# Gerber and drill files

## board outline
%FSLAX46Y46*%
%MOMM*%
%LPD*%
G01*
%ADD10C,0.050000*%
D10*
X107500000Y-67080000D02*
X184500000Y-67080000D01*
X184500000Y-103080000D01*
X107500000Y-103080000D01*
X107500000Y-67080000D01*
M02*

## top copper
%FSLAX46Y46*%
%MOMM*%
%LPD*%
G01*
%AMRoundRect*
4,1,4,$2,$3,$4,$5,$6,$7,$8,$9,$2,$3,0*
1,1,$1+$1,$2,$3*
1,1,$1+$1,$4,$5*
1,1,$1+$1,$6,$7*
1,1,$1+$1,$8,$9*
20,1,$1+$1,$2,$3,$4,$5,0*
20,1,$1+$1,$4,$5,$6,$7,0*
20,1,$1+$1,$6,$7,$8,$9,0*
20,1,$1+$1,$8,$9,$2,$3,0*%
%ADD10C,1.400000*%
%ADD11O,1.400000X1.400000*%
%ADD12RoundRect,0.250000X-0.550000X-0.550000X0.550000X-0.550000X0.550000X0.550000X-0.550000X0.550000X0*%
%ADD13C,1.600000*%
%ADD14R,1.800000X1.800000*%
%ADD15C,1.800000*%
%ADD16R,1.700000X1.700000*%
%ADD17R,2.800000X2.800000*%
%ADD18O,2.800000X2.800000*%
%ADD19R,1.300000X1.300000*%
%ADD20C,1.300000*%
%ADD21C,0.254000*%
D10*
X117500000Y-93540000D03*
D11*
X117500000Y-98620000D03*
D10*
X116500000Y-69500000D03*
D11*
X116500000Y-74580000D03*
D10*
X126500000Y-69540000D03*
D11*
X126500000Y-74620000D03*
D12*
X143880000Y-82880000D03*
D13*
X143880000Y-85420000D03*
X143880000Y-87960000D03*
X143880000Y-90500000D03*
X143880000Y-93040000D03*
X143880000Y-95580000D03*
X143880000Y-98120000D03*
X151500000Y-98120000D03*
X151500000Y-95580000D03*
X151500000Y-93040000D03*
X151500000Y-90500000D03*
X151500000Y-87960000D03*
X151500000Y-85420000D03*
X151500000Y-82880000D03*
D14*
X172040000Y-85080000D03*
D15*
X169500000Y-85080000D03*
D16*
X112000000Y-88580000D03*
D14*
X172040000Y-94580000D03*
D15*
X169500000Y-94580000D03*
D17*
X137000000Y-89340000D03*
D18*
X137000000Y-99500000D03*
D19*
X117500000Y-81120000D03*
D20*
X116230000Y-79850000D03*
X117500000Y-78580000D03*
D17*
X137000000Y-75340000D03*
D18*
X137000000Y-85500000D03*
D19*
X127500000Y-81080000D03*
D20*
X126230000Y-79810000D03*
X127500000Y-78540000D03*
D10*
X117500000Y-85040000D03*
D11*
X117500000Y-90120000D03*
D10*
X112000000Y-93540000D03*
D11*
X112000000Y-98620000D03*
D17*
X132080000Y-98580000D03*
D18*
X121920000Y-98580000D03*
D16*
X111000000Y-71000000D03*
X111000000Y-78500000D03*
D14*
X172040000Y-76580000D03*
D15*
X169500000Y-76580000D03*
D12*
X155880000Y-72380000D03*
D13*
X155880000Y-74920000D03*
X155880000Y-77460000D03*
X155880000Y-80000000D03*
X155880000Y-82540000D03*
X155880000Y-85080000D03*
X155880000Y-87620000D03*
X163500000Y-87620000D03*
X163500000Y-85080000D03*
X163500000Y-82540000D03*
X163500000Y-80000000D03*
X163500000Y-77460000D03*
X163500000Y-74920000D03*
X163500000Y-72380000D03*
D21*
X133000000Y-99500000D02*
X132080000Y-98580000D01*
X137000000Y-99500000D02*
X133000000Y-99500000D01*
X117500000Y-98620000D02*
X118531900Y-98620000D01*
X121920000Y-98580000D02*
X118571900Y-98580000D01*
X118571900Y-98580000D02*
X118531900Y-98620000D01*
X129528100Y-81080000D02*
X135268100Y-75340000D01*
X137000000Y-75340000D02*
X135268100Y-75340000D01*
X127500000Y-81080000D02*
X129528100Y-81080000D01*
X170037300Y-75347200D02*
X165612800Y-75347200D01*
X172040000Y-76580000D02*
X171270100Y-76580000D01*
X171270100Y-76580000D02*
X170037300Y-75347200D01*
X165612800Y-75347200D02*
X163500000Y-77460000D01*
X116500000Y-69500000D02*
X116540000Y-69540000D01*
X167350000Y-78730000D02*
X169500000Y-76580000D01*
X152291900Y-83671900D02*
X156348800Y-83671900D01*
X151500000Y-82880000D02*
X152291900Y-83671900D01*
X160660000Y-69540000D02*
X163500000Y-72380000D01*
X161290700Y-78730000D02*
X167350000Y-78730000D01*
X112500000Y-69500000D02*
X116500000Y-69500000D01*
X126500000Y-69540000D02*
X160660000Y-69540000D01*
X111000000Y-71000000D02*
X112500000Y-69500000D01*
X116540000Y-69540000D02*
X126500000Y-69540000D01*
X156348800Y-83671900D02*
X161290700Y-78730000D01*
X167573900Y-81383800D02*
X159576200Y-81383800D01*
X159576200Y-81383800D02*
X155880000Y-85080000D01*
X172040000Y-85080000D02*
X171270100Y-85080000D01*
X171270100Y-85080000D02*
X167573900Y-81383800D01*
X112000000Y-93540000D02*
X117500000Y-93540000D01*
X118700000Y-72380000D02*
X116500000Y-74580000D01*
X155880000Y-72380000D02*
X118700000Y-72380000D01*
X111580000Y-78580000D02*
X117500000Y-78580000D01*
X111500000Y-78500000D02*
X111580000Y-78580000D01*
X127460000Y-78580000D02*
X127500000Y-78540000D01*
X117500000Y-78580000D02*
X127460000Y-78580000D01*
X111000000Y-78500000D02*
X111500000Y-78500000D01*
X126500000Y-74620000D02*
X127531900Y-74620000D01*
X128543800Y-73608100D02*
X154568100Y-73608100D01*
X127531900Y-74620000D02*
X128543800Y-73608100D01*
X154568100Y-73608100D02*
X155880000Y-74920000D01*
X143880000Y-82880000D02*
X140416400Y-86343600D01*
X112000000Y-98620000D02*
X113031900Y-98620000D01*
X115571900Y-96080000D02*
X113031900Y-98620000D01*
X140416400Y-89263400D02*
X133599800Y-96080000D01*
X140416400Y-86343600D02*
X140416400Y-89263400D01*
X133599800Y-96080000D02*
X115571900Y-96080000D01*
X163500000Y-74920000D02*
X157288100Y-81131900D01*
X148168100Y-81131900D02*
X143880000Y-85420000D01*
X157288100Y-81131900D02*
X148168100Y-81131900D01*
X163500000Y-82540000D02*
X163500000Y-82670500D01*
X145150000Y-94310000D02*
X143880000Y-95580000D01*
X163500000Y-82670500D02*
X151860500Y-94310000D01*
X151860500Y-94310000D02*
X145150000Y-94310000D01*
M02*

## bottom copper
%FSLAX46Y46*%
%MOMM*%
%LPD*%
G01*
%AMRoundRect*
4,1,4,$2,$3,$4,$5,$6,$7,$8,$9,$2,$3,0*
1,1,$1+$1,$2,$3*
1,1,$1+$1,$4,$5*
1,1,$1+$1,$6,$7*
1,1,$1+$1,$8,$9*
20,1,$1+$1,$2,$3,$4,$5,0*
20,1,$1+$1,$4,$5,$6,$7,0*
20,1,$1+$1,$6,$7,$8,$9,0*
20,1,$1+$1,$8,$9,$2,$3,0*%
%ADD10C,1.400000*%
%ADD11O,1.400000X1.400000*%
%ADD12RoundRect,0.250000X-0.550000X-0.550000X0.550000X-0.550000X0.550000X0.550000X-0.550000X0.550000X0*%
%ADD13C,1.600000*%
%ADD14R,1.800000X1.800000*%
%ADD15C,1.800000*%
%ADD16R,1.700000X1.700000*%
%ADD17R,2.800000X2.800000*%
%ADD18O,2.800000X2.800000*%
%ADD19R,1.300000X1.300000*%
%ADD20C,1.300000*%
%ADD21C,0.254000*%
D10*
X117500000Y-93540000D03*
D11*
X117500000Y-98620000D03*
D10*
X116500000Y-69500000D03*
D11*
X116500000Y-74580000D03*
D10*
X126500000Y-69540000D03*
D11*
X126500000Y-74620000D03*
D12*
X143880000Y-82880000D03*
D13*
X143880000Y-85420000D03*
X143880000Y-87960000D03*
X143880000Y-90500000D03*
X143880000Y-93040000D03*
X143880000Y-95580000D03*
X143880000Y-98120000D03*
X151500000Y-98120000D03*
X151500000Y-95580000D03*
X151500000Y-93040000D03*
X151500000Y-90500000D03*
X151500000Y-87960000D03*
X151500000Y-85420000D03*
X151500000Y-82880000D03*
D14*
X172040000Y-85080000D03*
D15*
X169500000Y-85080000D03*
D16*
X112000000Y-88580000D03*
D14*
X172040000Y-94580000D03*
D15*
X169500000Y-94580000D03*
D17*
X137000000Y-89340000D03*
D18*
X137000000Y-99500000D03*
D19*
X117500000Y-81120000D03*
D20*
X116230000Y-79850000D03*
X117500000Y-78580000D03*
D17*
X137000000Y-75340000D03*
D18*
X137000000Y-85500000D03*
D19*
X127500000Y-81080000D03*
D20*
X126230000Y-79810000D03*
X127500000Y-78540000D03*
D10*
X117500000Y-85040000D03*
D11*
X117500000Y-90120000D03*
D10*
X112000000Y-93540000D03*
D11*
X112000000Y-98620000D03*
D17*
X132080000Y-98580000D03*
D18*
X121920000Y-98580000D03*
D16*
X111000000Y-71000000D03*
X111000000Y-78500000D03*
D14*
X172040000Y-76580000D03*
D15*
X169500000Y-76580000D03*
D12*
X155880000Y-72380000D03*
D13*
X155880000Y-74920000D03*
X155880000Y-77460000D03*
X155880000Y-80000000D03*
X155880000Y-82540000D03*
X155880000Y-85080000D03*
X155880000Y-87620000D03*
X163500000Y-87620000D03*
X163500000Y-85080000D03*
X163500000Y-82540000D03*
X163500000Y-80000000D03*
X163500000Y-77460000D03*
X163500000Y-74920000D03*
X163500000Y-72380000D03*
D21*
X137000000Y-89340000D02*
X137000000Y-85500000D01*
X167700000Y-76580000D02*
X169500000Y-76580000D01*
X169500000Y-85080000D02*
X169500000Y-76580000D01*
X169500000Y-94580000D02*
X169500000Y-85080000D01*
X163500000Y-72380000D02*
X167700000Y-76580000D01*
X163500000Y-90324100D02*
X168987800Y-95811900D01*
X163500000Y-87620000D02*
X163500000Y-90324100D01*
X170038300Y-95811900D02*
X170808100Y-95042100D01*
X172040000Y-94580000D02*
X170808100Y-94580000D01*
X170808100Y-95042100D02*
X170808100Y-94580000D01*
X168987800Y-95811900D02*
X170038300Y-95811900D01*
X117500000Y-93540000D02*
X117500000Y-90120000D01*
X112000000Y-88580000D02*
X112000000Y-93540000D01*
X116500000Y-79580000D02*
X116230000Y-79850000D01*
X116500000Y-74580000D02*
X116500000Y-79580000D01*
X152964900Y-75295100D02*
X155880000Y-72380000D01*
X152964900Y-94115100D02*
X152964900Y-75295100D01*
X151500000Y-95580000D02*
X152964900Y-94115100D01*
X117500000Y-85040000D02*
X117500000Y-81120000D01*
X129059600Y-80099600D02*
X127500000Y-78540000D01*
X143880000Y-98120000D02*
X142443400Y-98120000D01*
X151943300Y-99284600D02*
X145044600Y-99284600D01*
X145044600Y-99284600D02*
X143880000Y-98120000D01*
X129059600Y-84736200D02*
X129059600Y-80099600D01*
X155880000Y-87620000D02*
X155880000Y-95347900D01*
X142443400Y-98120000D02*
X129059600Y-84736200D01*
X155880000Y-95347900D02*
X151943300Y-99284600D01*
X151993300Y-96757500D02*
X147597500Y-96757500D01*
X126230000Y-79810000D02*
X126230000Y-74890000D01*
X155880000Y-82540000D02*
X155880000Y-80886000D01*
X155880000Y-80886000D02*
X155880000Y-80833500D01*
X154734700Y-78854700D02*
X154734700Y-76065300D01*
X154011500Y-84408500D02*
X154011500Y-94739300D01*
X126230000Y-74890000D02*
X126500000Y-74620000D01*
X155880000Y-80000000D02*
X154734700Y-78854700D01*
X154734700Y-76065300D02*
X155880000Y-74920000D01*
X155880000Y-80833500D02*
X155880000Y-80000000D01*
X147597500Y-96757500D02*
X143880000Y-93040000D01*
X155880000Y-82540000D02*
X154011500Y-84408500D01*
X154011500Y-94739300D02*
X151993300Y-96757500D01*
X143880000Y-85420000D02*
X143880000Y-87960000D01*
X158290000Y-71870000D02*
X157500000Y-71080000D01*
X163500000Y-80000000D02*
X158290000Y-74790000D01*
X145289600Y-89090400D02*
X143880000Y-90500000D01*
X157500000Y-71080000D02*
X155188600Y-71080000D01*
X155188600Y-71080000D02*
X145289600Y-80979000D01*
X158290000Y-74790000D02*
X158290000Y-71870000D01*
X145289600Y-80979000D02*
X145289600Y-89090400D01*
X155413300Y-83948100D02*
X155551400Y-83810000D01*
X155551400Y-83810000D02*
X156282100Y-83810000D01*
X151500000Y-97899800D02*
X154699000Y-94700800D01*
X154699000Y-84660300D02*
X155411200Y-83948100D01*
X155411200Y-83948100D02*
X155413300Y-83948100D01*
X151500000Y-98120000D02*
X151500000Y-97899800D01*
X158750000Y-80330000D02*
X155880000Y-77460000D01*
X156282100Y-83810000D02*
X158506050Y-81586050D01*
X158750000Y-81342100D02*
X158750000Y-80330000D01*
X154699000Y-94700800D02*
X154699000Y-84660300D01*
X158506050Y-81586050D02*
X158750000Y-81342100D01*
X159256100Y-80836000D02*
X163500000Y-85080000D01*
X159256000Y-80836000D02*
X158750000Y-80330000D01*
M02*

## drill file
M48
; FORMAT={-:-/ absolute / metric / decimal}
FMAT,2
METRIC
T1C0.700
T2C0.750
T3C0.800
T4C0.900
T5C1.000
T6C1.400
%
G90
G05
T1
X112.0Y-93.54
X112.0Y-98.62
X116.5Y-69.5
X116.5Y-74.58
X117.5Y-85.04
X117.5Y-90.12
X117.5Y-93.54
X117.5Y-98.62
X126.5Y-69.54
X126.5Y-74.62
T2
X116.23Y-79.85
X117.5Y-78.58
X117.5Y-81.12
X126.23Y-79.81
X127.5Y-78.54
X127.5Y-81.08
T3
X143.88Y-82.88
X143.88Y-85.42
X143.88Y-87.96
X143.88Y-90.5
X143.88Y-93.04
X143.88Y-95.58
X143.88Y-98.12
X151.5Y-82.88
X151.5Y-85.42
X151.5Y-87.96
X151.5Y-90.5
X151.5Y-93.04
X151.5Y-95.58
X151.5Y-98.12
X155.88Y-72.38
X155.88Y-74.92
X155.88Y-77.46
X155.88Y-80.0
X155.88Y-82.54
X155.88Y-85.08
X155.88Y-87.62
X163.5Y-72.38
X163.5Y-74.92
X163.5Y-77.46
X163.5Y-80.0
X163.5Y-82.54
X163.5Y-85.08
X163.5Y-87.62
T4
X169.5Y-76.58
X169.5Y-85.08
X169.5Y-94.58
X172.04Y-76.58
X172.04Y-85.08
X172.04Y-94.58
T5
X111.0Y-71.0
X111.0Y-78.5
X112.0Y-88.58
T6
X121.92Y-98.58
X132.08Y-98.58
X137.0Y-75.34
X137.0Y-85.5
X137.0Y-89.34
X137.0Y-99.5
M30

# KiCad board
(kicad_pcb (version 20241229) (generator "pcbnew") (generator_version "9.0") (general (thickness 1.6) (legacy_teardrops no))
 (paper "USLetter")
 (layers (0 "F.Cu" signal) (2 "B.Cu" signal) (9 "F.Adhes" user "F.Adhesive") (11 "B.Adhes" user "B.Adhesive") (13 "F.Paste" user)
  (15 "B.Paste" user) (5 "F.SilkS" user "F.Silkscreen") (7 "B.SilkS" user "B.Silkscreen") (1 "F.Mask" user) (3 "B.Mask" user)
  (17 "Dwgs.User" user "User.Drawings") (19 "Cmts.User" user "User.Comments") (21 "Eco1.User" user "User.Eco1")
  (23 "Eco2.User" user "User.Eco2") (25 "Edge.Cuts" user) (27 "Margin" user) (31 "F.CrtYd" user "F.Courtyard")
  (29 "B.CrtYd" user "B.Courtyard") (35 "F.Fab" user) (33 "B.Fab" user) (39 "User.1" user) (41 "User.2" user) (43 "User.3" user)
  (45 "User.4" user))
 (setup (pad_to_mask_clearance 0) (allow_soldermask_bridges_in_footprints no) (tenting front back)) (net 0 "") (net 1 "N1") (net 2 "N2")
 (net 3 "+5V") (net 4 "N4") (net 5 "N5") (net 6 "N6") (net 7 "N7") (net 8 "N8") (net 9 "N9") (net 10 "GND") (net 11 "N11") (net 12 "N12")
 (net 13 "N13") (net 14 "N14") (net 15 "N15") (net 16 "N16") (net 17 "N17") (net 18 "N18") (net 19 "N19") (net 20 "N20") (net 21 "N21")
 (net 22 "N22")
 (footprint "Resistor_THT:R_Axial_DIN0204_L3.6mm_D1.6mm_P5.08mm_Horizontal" (layer "F.Cu") (at 117.5 93.54 -90)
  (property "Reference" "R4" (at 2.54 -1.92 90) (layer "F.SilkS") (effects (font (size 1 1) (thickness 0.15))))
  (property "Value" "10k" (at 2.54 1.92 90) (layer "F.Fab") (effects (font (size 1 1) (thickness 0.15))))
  (pad "1" thru_hole circle (at 0 0 270) (size 1.4 1.4) (drill 0.7) (layers "*.Cu" "*.Mask") (remove_unused_layers no) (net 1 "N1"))
  (pad "2" thru_hole oval (at 5.08 0 270) (size 1.4 1.4) (drill 0.7) (layers "*.Cu" "*.Mask") (remove_unused_layers no) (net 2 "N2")))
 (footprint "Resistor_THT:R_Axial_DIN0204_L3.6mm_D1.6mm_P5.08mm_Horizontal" (layer "F.Cu") (at 116.5 69.5 -90)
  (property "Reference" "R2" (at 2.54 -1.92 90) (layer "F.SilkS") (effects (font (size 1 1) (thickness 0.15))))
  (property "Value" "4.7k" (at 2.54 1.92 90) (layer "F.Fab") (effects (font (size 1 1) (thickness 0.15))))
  (pad "1" thru_hole circle (at 0 0 270) (size 1.4 1.4) (drill 0.7) (layers "*.Cu" "*.Mask") (remove_unused_layers no) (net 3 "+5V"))
  (pad "2" thru_hole oval (at 5.08 0 270) (size 1.4 1.4) (drill 0.7) (layers "*.Cu" "*.Mask") (remove_unused_layers no) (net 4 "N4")))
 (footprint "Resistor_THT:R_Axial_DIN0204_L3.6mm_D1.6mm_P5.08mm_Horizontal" (layer "F.Cu") (at 126.5 69.54 -90)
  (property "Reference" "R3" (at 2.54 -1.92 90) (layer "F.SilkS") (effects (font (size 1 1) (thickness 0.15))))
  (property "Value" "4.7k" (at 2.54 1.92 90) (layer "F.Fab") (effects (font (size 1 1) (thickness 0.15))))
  (pad "1" thru_hole circle (at 0 0 270) (size 1.4 1.4) (drill 0.7) (layers "*.Cu" "*.Mask") (remove_unused_layers no) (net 3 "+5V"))
  (pad "2" thru_hole oval (at 5.08 0 270) (size 1.4 1.4) (drill 0.7) (layers "*.Cu" "*.Mask") (remove_unused_layers no) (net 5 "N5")))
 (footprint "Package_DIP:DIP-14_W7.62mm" (layer "F.Cu") (at 143.88 82.88)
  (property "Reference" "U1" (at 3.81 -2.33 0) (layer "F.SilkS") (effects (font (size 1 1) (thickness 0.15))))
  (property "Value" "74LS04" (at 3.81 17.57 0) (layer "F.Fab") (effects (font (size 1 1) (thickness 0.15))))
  (pad "1" thru_hole roundrect (at 0 0) (size 1.6 1.6) (drill 0.8) (layers "*.Cu" "*.Mask") (remove_unused_layers no)
   (roundrect_rratio 0.15625) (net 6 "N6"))
  (pad "2" thru_hole circle (at 0 2.54) (size 1.6 1.6) (drill 0.8) (layers "*.Cu" "*.Mask") (remove_unused_layers no) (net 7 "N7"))
  (pad "3" thru_hole circle (at 0 5.08) (size 1.6 1.6) (drill 0.8) (layers "*.Cu" "*.Mask") (remove_unused_layers no) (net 7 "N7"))
  (pad "4" thru_hole circle (at 0 7.62) (size 1.6 1.6) (drill 0.8) (layers "*.Cu" "*.Mask") (remove_unused_layers no) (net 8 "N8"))
  (pad "5" thru_hole circle (at 0 10.16) (size 1.6 1.6) (drill 0.8) (layers "*.Cu" "*.Mask") (remove_unused_layers no) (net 5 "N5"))
  (pad "6" thru_hole circle (at 0 12.7) (size 1.6 1.6) (drill 0.8) (layers "*.Cu" "*.Mask") (remove_unused_layers no) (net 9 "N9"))
  (pad "7" thru_hole circle (at 0 15.24) (size 1.6 1.6) (drill 0.8) (layers "*.Cu" "*.Mask") (remove_unused_layers no) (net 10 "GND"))
  (pad "8" thru_hole circle (at 7.62 15.24) (size 1.6 1.6) (drill 0.8) (layers "*.Cu" "*.Mask") (remove_unused_layers no) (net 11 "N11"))
  (pad "9" thru_hole circle (at 7.62 12.7) (size 1.6 1.6) (drill 0.8) (layers "*.Cu" "*.Mask") (remove_unused_layers no) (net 4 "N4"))
  (pad "10" thru_hole circle (at 7.62 10.16) (size 1.6 1.6) (drill 0.8) (layers "*.Cu" "*.Mask") (remove_unused_layers no) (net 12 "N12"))
  (pad "11" thru_hole circle (at 7.62 7.62) (size 1.6 1.6) (drill 0.8) (layers "*.Cu" "*.Mask") (remove_unused_layers no) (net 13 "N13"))
  (pad "12" thru_hole circle (at 7.62 5.08) (size 1.6 1.6) (drill 0.8) (layers "*.Cu" "*.Mask") (remove_unused_layers no) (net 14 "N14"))
  (pad "13" thru_hole circle (at 7.62 2.54) (size 1.6 1.6) (drill 0.8) (layers "*.Cu" "*.Mask") (remove_unused_layers no) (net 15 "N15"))
  (pad "14" thru_hole circle (at 7.62 0) (size 1.6 1.6) (drill 0.8) (layers "*.Cu" "*.Mask") (remove_unused_layers no) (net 3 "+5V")))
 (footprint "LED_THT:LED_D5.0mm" (layer "F.Cu") (at 172.04 85.08 180)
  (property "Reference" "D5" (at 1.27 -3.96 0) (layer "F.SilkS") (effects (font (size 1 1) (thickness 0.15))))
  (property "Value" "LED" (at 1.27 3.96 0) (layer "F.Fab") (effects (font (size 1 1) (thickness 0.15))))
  (pad "1" thru_hole rect (at 0 0 180) (size 1.8 1.8) (drill 0.9) (layers "*.Cu" "*.Mask") (remove_unused_layers no) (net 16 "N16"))
  (pad "2" thru_hole circle (at 2.54 0 180) (size 1.8 1.8) (drill 0.9) (layers "*.Cu" "*.Mask") (remove_unused_layers no) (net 3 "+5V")))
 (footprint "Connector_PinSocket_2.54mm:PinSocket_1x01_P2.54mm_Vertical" (layer "F.Cu") (at 112 88.58)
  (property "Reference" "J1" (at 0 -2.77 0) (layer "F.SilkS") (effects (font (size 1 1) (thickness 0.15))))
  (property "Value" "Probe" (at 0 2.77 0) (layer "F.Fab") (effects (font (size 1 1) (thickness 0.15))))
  (pad "1" thru_hole rect (at 0 0) (size 1.7 1.7) (drill 1) (layers "*.Cu" "*.Mask") (remove_unused_layers no) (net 1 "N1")))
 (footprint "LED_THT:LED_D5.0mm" (layer "F.Cu") (at 172.04 94.58 180)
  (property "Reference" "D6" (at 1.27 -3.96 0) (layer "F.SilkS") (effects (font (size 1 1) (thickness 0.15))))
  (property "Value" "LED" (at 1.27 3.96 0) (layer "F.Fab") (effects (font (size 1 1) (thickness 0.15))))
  (pad "1" thru_hole rect (at 0 0 180) (size 1.8 1.8) (drill 0.9) (layers "*.Cu" "*.Mask") (remove_unused_layers no) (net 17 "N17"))
  (pad "2" thru_hole circle (at 2.54 0 180) (size 1.8 1.8) (drill 0.9) (layers "*.Cu" "*.Mask") (remove_unused_layers no) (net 3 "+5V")))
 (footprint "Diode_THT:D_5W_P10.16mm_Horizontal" (layer "F.Cu") (at 137 89.34 -90)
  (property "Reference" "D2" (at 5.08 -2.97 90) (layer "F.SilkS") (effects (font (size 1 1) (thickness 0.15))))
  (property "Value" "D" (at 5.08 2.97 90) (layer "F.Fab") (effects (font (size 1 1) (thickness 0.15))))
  (pad "1" thru_hole rect (at 0 0 270) (size 2.8 2.8) (drill 1.4) (layers "*.Cu" "*.Mask") (remove_unused_layers no) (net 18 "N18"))
  (pad "2" thru_hole oval (at 10.16 0 270) (size 2.8 2.8) (drill 1.4) (layers "*.Cu" "*.Mask") (remove_unused_layers no) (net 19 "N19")))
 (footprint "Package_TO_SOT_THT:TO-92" (layer "F.Cu") (at 117.5 81.12 90)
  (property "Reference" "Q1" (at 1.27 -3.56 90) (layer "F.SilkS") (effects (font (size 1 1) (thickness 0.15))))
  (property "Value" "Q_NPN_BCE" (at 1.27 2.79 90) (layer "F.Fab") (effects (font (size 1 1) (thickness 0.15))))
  (pad "1" thru_hole rect (at 0 0 90) (size 1.3 1.3) (drill 0.75) (layers "*.Cu" "*.Mask") (remove_unused_layers no) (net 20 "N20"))
  (pad "2" thru_hole circle (at 1.27 -1.27 90) (size 1.3 1.3) (drill 0.75) (layers "*.Cu" "*.Mask") (remove_unused_layers no) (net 4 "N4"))
  (pad "3" thru_hole circle (at 2.54 0 90) (size 1.3 1.3) (drill 0.75) (layers "*.Cu" "*.Mask") (remove_unused_layers no) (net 10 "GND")))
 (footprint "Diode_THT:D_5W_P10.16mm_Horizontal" (layer "F.Cu") (at 137 75.34 -90)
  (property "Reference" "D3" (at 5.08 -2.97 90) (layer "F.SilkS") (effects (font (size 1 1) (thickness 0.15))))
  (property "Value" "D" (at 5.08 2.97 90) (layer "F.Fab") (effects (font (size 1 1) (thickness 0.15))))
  (pad "1" thru_hole rect (at 0 0 270) (size 2.8 2.8) (drill 1.4) (layers "*.Cu" "*.Mask") (remove_unused_layers no) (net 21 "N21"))
  (pad "2" thru_hole oval (at 10.16 0 270) (size 2.8 2.8) (drill 1.4) (layers "*.Cu" "*.Mask") (remove_unused_layers no) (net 18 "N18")))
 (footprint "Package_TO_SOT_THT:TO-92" (layer "F.Cu") (at 127.5 81.08 90)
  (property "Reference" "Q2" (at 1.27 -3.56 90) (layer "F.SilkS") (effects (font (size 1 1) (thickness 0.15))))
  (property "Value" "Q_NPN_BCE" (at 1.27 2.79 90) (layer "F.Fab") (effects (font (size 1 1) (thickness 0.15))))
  (pad "1" thru_hole rect (at 0 0 90) (size 1.3 1.3) (drill 0.75) (layers "*.Cu" "*.Mask") (remove_unused_layers no) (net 21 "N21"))
  (pad "2" thru_hole circle (at 1.27 -1.27 90) (size 1.3 1.3) (drill 0.75) (layers "*.Cu" "*.Mask") (remove_unused_layers no) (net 5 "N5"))
  (pad "3" thru_hole circle (at 2.54 0 90) (size 1.3 1.3) (drill 0.75) (layers "*.Cu" "*.Mask") (remove_unused_layers no) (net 10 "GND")))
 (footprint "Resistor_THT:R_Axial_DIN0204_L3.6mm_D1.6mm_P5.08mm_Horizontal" (layer "F.Cu") (at 117.5 85.04 -90)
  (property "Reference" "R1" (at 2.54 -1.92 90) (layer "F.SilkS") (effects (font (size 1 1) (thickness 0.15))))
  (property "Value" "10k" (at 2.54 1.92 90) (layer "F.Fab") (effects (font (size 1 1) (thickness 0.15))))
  (pad "1" thru_hole circle (at 0 0 270) (size 1.4 1.4) (drill 0.7) (layers "*.Cu" "*.Mask") (remove_unused_layers no) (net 20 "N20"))
  (pad "2" thru_hole oval (at 5.08 0 270) (size 1.4 1.4) (drill 0.7) (layers "*.Cu" "*.Mask") (remove_unused_layers no) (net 1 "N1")))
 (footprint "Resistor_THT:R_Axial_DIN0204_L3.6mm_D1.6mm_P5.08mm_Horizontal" (layer "F.Cu") (at 112 93.54 -90)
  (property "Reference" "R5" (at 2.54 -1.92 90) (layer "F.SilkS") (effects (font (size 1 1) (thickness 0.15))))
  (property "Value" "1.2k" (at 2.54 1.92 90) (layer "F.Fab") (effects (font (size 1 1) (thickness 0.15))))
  (pad "1" thru_hole circle (at 0 0 270) (size 1.4 1.4) (drill 0.7) (layers "*.Cu" "*.Mask") (remove_unused_layers no) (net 1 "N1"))
  (pad "2" thru_hole oval (at 5.08 0 270) (size 1.4 1.4) (drill 0.7) (layers "*.Cu" "*.Mask") (remove_unused_layers no) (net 6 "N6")))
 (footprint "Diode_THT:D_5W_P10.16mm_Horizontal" (layer "F.Cu") (at 132.08 98.58 180)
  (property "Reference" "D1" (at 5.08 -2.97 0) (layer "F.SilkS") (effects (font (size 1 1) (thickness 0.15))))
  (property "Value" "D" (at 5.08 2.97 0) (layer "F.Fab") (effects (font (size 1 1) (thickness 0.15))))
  (pad "1" thru_hole rect (at 0 0 180) (size 2.8 2.8) (drill 1.4) (layers "*.Cu" "*.Mask") (remove_unused_layers no) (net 19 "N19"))
  (pad "2" thru_hole oval (at 10.16 0 180) (size 2.8 2.8) (drill 1.4) (layers "*.Cu" "*.Mask") (remove_unused_layers no) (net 2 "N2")))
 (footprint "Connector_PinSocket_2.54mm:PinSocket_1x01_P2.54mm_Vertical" (layer "F.Cu") (at 111 71)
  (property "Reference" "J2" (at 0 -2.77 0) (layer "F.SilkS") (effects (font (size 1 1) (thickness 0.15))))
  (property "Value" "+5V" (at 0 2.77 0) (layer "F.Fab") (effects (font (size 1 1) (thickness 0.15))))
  (pad "1" thru_hole rect (at 0 0) (size 1.7 1.7) (drill 1) (layers "*.Cu" "*.Mask") (remove_unused_layers no) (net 3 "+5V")))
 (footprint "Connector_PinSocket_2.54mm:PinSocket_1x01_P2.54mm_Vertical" (layer "F.Cu") (at 111 78.5)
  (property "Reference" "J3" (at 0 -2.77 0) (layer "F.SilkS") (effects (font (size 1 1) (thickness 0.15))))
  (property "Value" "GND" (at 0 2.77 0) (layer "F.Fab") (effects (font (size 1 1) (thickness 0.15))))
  (pad "1" thru_hole rect (at 0 0) (size 1.7 1.7) (drill 1) (layers "*.Cu" "*.Mask") (remove_unused_layers no) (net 10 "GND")))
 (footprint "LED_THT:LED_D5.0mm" (layer "F.Cu") (at 172.04 76.58 180)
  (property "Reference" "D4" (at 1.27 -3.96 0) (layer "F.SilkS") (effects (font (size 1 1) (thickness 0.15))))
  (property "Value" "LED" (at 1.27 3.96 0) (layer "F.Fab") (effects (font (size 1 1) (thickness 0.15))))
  (pad "1" thru_hole rect (at 0 0 180) (size 1.8 1.8) (drill 0.9) (layers "*.Cu" "*.Mask") (remove_unused_layers no) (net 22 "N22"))
  (pad "2" thru_hole circle (at 2.54 0 180) (size 1.8 1.8) (drill 0.9) (layers "*.Cu" "*.Mask") (remove_unused_layers no) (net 3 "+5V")))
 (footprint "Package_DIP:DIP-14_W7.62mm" (layer "F.Cu") (at 155.88 72.38)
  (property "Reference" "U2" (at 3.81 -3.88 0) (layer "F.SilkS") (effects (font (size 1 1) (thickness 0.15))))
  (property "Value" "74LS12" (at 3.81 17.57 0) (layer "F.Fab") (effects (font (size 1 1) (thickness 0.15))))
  (pad "1" thru_hole roundrect (at 0 0) (size 1.6 1.6) (drill 0.8) (layers "*.Cu" "*.Mask") (remove_unused_layers no)
   (roundrect_rratio 0.15625) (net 4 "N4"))
  (pad "2" thru_hole circle (at 0 2.54) (size 1.6 1.6) (drill 0.8) (layers "*.Cu" "*.Mask") (remove_unused_layers no) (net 5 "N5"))
  (pad "3" thru_hole circle (at 0 5.08) (size 1.6 1.6) (drill 0.8) (layers "*.Cu" "*.Mask") (remove_unused_layers no) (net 11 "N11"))
  (pad "4" thru_hole circle (at 0 7.62) (size 1.6 1.6) (drill 0.8) (layers "*.Cu" "*.Mask") (remove_unused_layers no) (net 5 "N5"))
  (pad "5" thru_hole circle (at 0 10.16) (size 1.6 1.6) (drill 0.8) (layers "*.Cu" "*.Mask") (remove_unused_layers no) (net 5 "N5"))
  (pad "6" thru_hole circle (at 0 12.7) (size 1.6 1.6) (drill 0.8) (layers "*.Cu" "*.Mask") (remove_unused_layers no) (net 16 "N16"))
  (pad "7" thru_hole circle (at 0 15.24) (size 1.6 1.6) (drill 0.8) (layers "*.Cu" "*.Mask") (remove_unused_layers no) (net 10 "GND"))
  (pad "8" thru_hole circle (at 7.62 15.24) (size 1.6 1.6) (drill 0.8) (layers "*.Cu" "*.Mask") (remove_unused_layers no) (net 17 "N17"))
  (pad "9" thru_hole circle (at 7.62 12.7) (size 1.6 1.6) (drill 0.8) (layers "*.Cu" "*.Mask") (remove_unused_layers no) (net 11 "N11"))
  (pad "10" thru_hole circle (at 7.62 10.16) (size 1.6 1.6) (drill 0.8) (layers "*.Cu" "*.Mask") (remove_unused_layers no) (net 9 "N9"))
  (pad "11" thru_hole circle (at 7.62 7.62) (size 1.6 1.6) (drill 0.8) (layers "*.Cu" "*.Mask") (remove_unused_layers no) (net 8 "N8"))
  (pad "12" thru_hole circle (at 7.62 5.08) (size 1.6 1.6) (drill 0.8) (layers "*.Cu" "*.Mask") (remove_unused_layers no) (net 22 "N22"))
  (pad "13" thru_hole circle (at 7.62 2.54) (size 1.6 1.6) (drill 0.8) (layers "*.Cu" "*.Mask") (remove_unused_layers no) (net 7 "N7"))
  (pad "14" thru_hole circle (at 7.62 0) (size 1.6 1.6) (drill 0.8) (layers "*.Cu" "*.Mask") (remove_unused_layers no) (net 3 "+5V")))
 (gr_rect (start 107.5 67.08) (end 184.5 103.08) (stroke (width 0.05) (type default)) (fill no) (layer "Edge.Cuts"))
 (segment (start 133 99.5) (end 132.08 98.58) (width 0.254) (layer "F.Cu") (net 19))
 (segment (start 137 99.5) (end 133 99.5) (width 0.254) (layer "F.Cu") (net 19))
 (segment (start 117.5 98.62) (end 118.5319 98.62) (width 0.254) (layer "F.Cu") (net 2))
 (segment (start 121.92 98.58) (end 118.5719 98.58) (width 0.254) (layer "F.Cu") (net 2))
 (segment (start 118.5719 98.58) (end 118.5319 98.62) (width 0.254) (layer "F.Cu") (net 2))
 (segment (start 137 89.34) (end 137 85.5) (width 0.254) (layer "B.Cu") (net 18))
 (segment (start 129.5281 81.08) (end 135.2681 75.34) (width 0.254) (layer "F.Cu") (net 21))
 (segment (start 137 75.34) (end 135.2681 75.34) (width 0.254) (layer "F.Cu") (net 21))
 (segment (start 127.5 81.08) (end 129.5281 81.08) (width 0.254) (layer "F.Cu") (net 21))
 (segment (start 170.0373 75.3472) (end 165.6128 75.3472) (width 0.254) (layer "F.Cu") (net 22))
 (segment (start 172.04 76.58) (end 171.2701 76.58) (width 0.254) (layer "F.Cu") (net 22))
 (segment (start 171.2701 76.58) (end 170.0373 75.3472) (width 0.254) (layer "F.Cu") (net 22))
 (segment (start 165.6128 75.3472) (end 163.5 77.46) (width 0.254) (layer "F.Cu") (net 22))
 (segment (start 116.5 69.5) (end 116.54 69.54) (width 0.254) (layer "F.Cu") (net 3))
 (segment (start 167.35 78.73) (end 169.5 76.58) (width 0.254) (layer "F.Cu") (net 3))
 (segment (start 152.2919 83.6719) (end 156.3488 83.6719) (width 0.254) (layer "F.Cu") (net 3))
 (segment (start 151.5 82.88) (end 152.2919 83.6719) (width 0.254) (layer "F.Cu") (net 3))
 (segment (start 160.66 69.54) (end 163.5 72.38) (width 0.254) (layer "F.Cu") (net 3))
 (segment (start 161.2907 78.73) (end 167.35 78.73) (width 0.254) (layer "F.Cu") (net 3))
 (segment (start 112.5 69.5) (end 116.5 69.5) (width 0.254) (layer "F.Cu") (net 3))
 (segment (start 126.5 69.54) (end 160.66 69.54) (width 0.254) (layer "F.Cu") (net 3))
 (segment (start 111 71) (end 112.5 69.5) (width 0.254) (layer "F.Cu") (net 3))
 (segment (start 116.54 69.54) (end 126.5 69.54) (width 0.254) (layer "F.Cu") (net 3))
 (segment (start 156.3488 83.6719) (end 161.2907 78.73) (width 0.254) (layer "F.Cu") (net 3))
 (segment (start 167.7 76.58) (end 169.5 76.58) (width 0.254) (layer "B.Cu") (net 3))
 (segment (start 169.5 85.08) (end 169.5 76.58) (width 0.254) (layer "B.Cu") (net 3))
 (segment (start 169.5 94.58) (end 169.5 85.08) (width 0.254) (layer "B.Cu") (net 3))
 (segment (start 163.5 72.38) (end 167.7 76.58) (width 0.254) (layer "B.Cu") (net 3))
 (segment (start 167.5739 81.3838) (end 159.5762 81.3838) (width 0.254) (layer "F.Cu") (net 16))
 (segment (start 159.5762 81.3838) (end 155.88 85.08) (width 0.254) (layer "F.Cu") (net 16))
 (segment (start 172.04 85.08) (end 171.2701 85.08) (width 0.254) (layer "F.Cu") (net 16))
 (segment (start 171.2701 85.08) (end 167.5739 81.3838) (width 0.254) (layer "F.Cu") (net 16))
 (segment (start 163.5 90.3241) (end 168.9878 95.8119) (width 0.254) (layer "B.Cu") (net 17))
 (segment (start 163.5 87.62) (end 163.5 90.3241) (width 0.254) (layer "B.Cu") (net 17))
 (segment (start 170.0383 95.8119) (end 170.8081 95.0421) (width 0.254) (layer "B.Cu") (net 17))
 (segment (start 172.04 94.58) (end 170.8081 94.58) (width 0.254) (layer "B.Cu") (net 17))
 (segment (start 170.8081 95.0421) (end 170.8081 94.58) (width 0.254) (layer "B.Cu") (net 17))
 (segment (start 168.9878 95.8119) (end 170.0383 95.8119) (width 0.254) (layer "B.Cu") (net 17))
 (segment (start 112 93.54) (end 117.5 93.54) (width 0.254) (layer "F.Cu") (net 1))
 (segment (start 117.5 93.54) (end 117.5 90.12) (width 0.254) (layer "B.Cu") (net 1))
 (segment (start 112 88.58) (end 112 93.54) (width 0.254) (layer "B.Cu") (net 1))
 (segment (start 118.7 72.38) (end 116.5 74.58) (width 0.254) (layer "F.Cu") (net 4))
 (segment (start 155.88 72.38) (end 118.7 72.38) (width 0.254) (layer "F.Cu") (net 4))
 (segment (start 116.5 79.58) (end 116.23 79.85) (width 0.254) (layer "B.Cu") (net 4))
 (segment (start 116.5 74.58) (end 116.5 79.58) (width 0.254) (layer "B.Cu") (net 4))
 (segment (start 152.9649 75.2951) (end 155.88 72.38) (width 0.254) (layer "B.Cu") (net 4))
 (segment (start 152.9649 94.1151) (end 152.9649 75.2951) (width 0.254) (layer "B.Cu") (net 4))
 (segment (start 151.5 95.58) (end 152.9649 94.1151) (width 0.254) (layer "B.Cu") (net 4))
 (segment (start 117.5 85.04) (end 117.5 81.12) (width 0.254) (layer "B.Cu") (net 20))
 (segment (start 111.58 78.58) (end 117.5 78.58) (width 0.254) (layer "F.Cu") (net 10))
 (segment (start 111.5 78.5) (end 111.58 78.58) (width 0.254) (layer "F.Cu") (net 10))
 (segment (start 127.46 78.58) (end 127.5 78.54) (width 0.254) (layer "F.Cu") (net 10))
 (segment (start 117.5 78.58) (end 127.46 78.58) (width 0.254) (layer "F.Cu") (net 10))
 (segment (start 111 78.5) (end 111.5 78.5) (width 0.254) (layer "F.Cu") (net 10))
 (segment (start 129.0596 80.0996) (end 127.5 78.54) (width 0.254) (layer "B.Cu") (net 10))
 (segment (start 143.88 98.12) (end 142.4434 98.12) (width 0.254) (layer "B.Cu") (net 10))
 (segment (start 151.9433 99.2846) (end 145.0446 99.2846) (width 0.254) (layer "B.Cu") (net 10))
 (segment (start 145.0446 99.2846) (end 143.88 98.12) (width 0.254) (layer "B.Cu") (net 10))
 (segment (start 129.0596 84.7362) (end 129.0596 80.0996) (width 0.254) (layer "B.Cu") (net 10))
 (segment (start 155.88 87.62) (end 155.88 95.3479) (width 0.254) (layer "B.Cu") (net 10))
 (segment (start 142.4434 98.12) (end 129.0596 84.7362) (width 0.254) (layer "B.Cu") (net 10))
 (segment (start 155.88 95.3479) (end 151.9433 99.2846) (width 0.254) (layer "B.Cu") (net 10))
 (segment (start 126.5 74.62) (end 127.5319 74.62) (width 0.254) (layer "F.Cu") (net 5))
 (segment (start 128.5438 73.6081) (end 154.5681 73.6081) (width 0.254) (layer "F.Cu") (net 5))
 (segment (start 127.5319 74.62) (end 128.5438 73.6081) (width 0.254) (layer "F.Cu") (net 5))
 (segment (start 154.5681 73.6081) (end 155.88 74.92) (width 0.254) (layer "F.Cu") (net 5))
 (segment (start 151.9933 96.7575) (end 147.5975 96.7575) (width 0.254) (layer "B.Cu") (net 5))
 (segment (start 126.23 79.81) (end 126.23 74.89) (width 0.254) (layer "B.Cu") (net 5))
 (segment (start 155.88 82.54) (end 155.88 80.886) (width 0.254) (layer "B.Cu") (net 5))
 (segment (start 155.88 80.886) (end 155.88 80.8335) (width 0.254) (layer "B.Cu") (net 5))
 (segment (start 154.7347 78.8547) (end 154.7347 76.0653) (width 0.254) (layer "B.Cu") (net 5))
 (segment (start 154.0115 84.4085) (end 154.0115 94.7393) (width 0.254) (layer "B.Cu") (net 5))
 (segment (start 126.23 74.89) (end 126.5 74.62) (width 0.254) (layer "B.Cu") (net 5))
 (segment (start 155.88 80) (end 154.7347 78.8547) (width 0.254) (layer "B.Cu") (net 5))
 (segment (start 154.7347 76.0653) (end 155.88 74.92) (width 0.254) (layer "B.Cu") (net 5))
 (segment (start 155.88 80.8335) (end 155.88 80) (width 0.254) (layer "B.Cu") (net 5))
 (segment (start 147.5975 96.7575) (end 143.88 93.04) (width 0.254) (layer "B.Cu") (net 5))
 (segment (start 155.88 82.54) (end 154.0115 84.4085) (width 0.254) (layer "B.Cu") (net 5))
 (segment (start 154.0115 94.7393) (end 151.9933 96.7575) (width 0.254) (layer "B.Cu") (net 5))
 (segment (start 143.88 82.88) (end 140.4164 86.3436) (width 0.254) (layer "F.Cu") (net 6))
 (segment (start 112 98.62) (end 113.0319 98.62) (width 0.254) (layer "F.Cu") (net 6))
 (segment (start 115.5719 96.08) (end 113.0319 98.62) (width 0.254) (layer "F.Cu") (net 6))
 (segment (start 140.4164 89.2634) (end 133.5998 96.08) (width 0.254) (layer "F.Cu") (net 6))
 (segment (start 140.4164 86.3436) (end 140.4164 89.2634) (width 0.254) (layer "F.Cu") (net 6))
 (segment (start 133.5998 96.08) (end 115.5719 96.08) (width 0.254) (layer "F.Cu") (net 6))
 (segment (start 163.5 74.92) (end 157.2881 81.1319) (width 0.254) (layer "F.Cu") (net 7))
 (segment (start 148.1681 81.1319) (end 143.88 85.42) (width 0.254) (layer "F.Cu") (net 7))
 (segment (start 157.2881 81.1319) (end 148.1681 81.1319) (width 0.254) (layer "F.Cu") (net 7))
 (segment (start 143.88 85.42) (end 143.88 87.96) (width 0.254) (layer "B.Cu") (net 7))
 (segment (start 163.5 82.54) (end 163.5 82.6705) (width 0.254) (layer "F.Cu") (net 9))
 (segment (start 145.15 94.31) (end 143.88 95.58) (width 0.254) (layer "F.Cu") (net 9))
 (segment (start 163.5 82.6705) (end 151.8605 94.31) (width 0.254) (layer "F.Cu") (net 9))
 (segment (start 151.8605 94.31) (end 145.15 94.31) (width 0.254) (layer "F.Cu") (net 9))
 (segment (start 158.29 71.87) (end 157.5 71.08) (width 0.254) (layer "B.Cu") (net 8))
 (segment (start 163.5 80) (end 158.29 74.79) (width 0.254) (layer "B.Cu") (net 8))
 (segment (start 145.2896 89.0904) (end 143.88 90.5) (width 0.254) (layer "B.Cu") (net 8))
 (segment (start 157.5 71.08) (end 155.1886 71.08) (width 0.254) (layer "B.Cu") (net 8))
 (segment (start 155.1886 71.08) (end 145.2896 80.979) (width 0.254) (layer "B.Cu") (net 8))
 (segment (start 158.29 74.79) (end 158.29 71.87) (width 0.254) (layer "B.Cu") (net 8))
 (segment (start 145.2896 80.979) (end 145.2896 89.0904) (width 0.254) (layer "B.Cu") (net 8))
 (segment (start 155.4133 83.9481) (end 155.5514 83.81) (width 0.254) (layer "B.Cu") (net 11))
 (segment (start 155.5514 83.81) (end 156.2821 83.81) (width 0.254) (layer "B.Cu") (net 11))
 (segment (start 151.5 97.8998) (end 154.699 94.7008) (width 0.254) (layer "B.Cu") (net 11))
 (segment (start 154.699 84.6603) (end 155.4112 83.9481) (width 0.254) (layer "B.Cu") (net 11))
 (segment (start 155.4112 83.9481) (end 155.4133 83.9481) (width 0.254) (layer "B.Cu") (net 11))
 (segment (start 151.5 98.12) (end 151.5 97.8998) (width 0.254) (layer "B.Cu") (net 11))
 (segment (start 158.75 80.33) (end 155.88 77.46) (width 0.254) (layer "B.Cu") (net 11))
 (segment (start 156.2821 83.81) (end 158.50605 81.58605) (width 0.254) (layer "B.Cu") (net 11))
 (segment (start 158.75 81.3421) (end 158.75 80.33) (width 0.254) (layer "B.Cu") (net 11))
 (segment (start 154.699 94.7008) (end 154.699 84.6603) (width 0.254) (layer "B.Cu") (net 11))
 (segment (start 158.50605 81.58605) (end 158.75 81.3421) (width 0.254) (layer "B.Cu") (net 11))
 (segment (start 159.2561 80.836) (end 163.5 85.08) (width 0.254) (layer "B.Cu") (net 11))
 (segment (start 159.256 80.836) (end 158.75 80.33) (width 0.254) (layer "B.Cu") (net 11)))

